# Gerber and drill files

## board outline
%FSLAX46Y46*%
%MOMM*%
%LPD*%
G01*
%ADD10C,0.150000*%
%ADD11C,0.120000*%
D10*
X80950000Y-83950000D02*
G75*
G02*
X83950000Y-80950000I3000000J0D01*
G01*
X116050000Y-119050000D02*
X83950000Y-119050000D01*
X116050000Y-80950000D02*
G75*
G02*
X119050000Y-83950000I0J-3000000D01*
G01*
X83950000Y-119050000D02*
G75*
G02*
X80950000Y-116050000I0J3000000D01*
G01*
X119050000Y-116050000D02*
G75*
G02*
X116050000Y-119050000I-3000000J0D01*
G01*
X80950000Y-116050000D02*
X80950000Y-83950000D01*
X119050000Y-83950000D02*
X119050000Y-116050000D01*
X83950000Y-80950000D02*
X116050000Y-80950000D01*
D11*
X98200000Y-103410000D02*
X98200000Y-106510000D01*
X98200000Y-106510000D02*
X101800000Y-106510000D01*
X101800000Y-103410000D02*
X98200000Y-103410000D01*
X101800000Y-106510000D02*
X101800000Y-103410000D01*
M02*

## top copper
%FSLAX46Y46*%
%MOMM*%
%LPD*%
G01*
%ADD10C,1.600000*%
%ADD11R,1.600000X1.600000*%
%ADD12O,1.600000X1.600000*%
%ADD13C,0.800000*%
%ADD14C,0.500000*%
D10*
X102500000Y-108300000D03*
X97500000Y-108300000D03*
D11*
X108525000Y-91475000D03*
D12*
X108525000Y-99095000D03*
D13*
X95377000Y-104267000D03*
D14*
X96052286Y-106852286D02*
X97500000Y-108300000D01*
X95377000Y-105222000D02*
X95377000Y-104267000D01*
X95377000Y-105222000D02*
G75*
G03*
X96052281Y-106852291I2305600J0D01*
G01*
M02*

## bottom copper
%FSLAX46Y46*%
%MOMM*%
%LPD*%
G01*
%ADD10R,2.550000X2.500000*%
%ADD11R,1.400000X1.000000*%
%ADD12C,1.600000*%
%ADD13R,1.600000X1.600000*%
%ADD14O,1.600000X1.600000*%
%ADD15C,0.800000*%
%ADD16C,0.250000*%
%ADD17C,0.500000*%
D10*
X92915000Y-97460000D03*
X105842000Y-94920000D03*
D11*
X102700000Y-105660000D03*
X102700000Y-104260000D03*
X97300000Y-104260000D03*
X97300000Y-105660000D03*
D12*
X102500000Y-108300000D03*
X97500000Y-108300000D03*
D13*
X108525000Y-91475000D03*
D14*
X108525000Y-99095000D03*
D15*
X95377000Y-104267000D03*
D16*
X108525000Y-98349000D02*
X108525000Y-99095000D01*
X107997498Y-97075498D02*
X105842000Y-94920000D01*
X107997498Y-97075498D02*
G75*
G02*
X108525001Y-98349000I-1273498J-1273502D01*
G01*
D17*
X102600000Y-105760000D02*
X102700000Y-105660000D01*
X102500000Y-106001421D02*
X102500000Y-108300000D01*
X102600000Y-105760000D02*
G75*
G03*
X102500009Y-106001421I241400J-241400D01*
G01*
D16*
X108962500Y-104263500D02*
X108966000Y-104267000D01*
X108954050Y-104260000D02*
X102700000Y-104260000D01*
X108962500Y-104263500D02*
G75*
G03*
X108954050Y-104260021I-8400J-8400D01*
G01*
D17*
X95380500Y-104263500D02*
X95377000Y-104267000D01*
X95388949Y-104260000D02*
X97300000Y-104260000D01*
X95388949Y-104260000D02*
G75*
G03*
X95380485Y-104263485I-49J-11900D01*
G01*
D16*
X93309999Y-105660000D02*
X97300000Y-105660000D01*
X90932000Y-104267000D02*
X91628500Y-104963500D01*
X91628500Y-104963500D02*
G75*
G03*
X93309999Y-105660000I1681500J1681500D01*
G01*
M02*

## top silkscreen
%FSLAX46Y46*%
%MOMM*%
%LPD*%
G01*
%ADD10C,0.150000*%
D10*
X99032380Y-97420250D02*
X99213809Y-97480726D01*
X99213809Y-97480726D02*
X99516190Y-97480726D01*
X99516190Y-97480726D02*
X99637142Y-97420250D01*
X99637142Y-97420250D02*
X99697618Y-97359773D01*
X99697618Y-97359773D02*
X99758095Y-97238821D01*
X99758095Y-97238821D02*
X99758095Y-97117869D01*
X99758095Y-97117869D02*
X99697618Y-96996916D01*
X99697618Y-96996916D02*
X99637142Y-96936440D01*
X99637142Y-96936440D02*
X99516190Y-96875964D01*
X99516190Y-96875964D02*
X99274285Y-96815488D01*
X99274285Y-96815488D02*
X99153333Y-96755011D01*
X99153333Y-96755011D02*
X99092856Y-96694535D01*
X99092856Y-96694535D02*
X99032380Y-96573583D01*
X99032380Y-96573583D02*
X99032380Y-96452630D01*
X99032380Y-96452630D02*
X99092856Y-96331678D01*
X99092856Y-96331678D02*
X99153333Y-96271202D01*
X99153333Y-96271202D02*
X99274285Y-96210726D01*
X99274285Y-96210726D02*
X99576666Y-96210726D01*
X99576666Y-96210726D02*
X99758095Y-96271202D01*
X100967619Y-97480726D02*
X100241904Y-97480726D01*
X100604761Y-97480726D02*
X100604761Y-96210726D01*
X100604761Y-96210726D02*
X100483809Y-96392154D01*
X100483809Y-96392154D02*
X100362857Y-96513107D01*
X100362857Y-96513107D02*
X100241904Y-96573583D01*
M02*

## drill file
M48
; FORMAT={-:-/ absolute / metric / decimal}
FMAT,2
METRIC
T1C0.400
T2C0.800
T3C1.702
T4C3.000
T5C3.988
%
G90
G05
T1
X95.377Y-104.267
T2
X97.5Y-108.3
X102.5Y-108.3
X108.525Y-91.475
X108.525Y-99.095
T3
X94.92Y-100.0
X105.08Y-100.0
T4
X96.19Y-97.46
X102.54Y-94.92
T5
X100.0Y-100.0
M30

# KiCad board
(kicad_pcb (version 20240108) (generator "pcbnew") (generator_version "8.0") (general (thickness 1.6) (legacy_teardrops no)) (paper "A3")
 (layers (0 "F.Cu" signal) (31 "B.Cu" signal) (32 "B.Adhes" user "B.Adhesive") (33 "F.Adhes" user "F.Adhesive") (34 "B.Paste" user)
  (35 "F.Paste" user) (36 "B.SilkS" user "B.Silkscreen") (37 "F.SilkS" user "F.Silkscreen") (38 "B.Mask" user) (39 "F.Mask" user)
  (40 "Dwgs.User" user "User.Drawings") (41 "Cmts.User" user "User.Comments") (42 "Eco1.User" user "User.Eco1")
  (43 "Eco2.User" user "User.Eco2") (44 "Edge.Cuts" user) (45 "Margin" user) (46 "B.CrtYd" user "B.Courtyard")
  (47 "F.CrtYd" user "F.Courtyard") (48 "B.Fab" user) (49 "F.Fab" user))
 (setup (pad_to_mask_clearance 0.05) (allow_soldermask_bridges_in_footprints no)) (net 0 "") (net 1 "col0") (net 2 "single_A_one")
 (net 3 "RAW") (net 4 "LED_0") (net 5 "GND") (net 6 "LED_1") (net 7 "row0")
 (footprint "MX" (layer "F.Cu") (at 100 100)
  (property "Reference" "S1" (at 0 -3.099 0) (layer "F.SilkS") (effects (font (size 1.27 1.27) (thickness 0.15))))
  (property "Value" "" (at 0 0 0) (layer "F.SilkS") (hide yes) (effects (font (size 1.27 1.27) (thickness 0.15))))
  (pad "" np_thru_hole circle (at -5.08 0) (size 1.7018 1.7018) (drill 1.7018) (layers "*.Cu" "*.Mask"))
  (pad "" np_thru_hole circle (at -3.81 -2.54) (size 3 3) (drill 3) (layers "*.Cu" "*.Mask"))
  (pad "" np_thru_hole circle (at 0 0) (size 3.9878 3.9878) (drill 3.9878) (layers "*.Cu" "*.Mask"))
  (pad "" np_thru_hole circle (at 2.54 -5.08) (size 3 3) (drill 3) (layers "*.Cu" "*.Mask"))
  (pad "" np_thru_hole circle (at 5.08 0) (size 1.7018 1.7018) (drill 1.7018) (layers "*.Cu" "*.Mask"))
  (pad "1" smd rect (at -7.085 -2.54) (size 2.55 2.5) (layers "B.Cu" "B.Paste" "B.Mask") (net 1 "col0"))
  (pad "2" smd rect (at 5.842 -5.08) (size 2.55 2.5) (layers "B.Cu" "B.Paste" "B.Mask") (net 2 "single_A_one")))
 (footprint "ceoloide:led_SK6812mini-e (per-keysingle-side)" (layer "B.Cu") (at 100 104.96)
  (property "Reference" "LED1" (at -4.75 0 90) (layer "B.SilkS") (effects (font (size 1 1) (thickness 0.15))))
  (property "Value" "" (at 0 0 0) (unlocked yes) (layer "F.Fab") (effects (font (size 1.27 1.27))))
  (fp_line (start -1.8 -1.55) (end -1.8 1.55) (stroke (width 0.12) (type solid)) (layer "Edge.Cuts"))
  (fp_line (start -1.8 1.55) (end 1.8 1.55) (stroke (width 0.12) (type solid)) (layer "Edge.Cuts"))
  (fp_line (start 1.8 -1.55) (end -1.8 -1.55) (stroke (width 0.12) (type solid)) (layer "Edge.Cuts"))
  (fp_line (start 1.8 1.55) (end 1.8 -1.55) (stroke (width 0.12) (type solid)) (layer "Edge.Cuts"))
  (pad "1" smd rect (at 2.7 0.7) (size 1.4 1) (layers "B.Cu" "B.Paste" "B.Mask") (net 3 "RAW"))
  (pad "2" smd rect (at 2.7 -0.7) (size 1.4 1) (layers "B.Cu" "B.Paste" "B.Mask") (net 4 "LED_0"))
  (pad "3" smd rect (at -2.7 -0.7) (size 1.4 1) (layers "B.Cu" "B.Paste" "B.Mask") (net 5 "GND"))
  (pad "4" smd rect (at -2.7 0.7) (size 1.4 1) (layers "B.Cu" "B.Paste" "B.Mask") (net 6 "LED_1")))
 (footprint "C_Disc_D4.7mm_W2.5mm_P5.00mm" (layer "B.Cu") (at 102.5 108.3 180)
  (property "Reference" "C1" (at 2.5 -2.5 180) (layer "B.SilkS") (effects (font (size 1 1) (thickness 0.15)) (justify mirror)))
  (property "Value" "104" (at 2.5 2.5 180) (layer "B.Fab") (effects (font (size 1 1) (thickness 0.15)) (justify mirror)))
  (pad "1" thru_hole circle (at 0 0) (size 1.6 1.6) (drill 0.8) (layers "*.Cu" "*.Mask") (remove_unused_layers no) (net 3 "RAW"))
  (pad "2" thru_hole circle (at 5 0) (size 1.6 1.6) (drill 0.8) (layers "*.Cu" "*.Mask") (remove_unused_layers no) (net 5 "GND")))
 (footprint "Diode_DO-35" (layer "B.Cu") (at 108.525 91.475 -90)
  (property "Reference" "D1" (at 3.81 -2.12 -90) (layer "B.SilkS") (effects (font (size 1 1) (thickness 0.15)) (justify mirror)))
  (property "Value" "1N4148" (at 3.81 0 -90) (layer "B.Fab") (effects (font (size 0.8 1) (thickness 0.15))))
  (pad "1" thru_hole rect (at 0 0 270) (size 1.6 1.6) (drill 0.8) (layers "*.Cu" "*.Mask") (remove_unused_layers no) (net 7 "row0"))
  (pad "2" thru_hole oval (at 7.62 0 270) (size 1.6 1.6) (drill 0.8) (layers "*.Cu" "*.Mask") (remove_unused_layers no)
   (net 2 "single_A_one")))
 (gr_arc (start 80.95 83.95) (mid 81.82868 81.82868) (end 83.95 80.95) (stroke (width 0.15) (type solid)) (layer "Edge.Cuts"))
 (gr_line (start 116.05 119.05) (end 83.95 119.05) (stroke (width 0.15) (type solid)) (layer "Edge.Cuts"))
 (gr_arc (start 116.05 80.95) (mid 118.17132 81.82868) (end 119.05 83.95) (stroke (width 0.15) (type solid)) (layer "Edge.Cuts"))
 (gr_arc (start 83.95 119.05) (mid 81.82868 118.17132) (end 80.95 116.05) (stroke (width 0.15) (type solid)) (layer "Edge.Cuts"))
 (gr_arc (start 119.05 116.05) (mid 118.17132 118.17132) (end 116.05 119.05) (stroke (width 0.15) (type solid)) (layer "Edge.Cuts"))
 (gr_line (start 80.95 116.05) (end 80.95 83.95) (stroke (width 0.15) (type solid)) (layer "Edge.Cuts"))
 (gr_line (start 119.05 83.95) (end 119.05 116.05) (stroke (width 0.15) (type solid)) (layer "Edge.Cuts"))
 (gr_line (start 83.95 80.95) (end 116.05 80.95) (stroke (width 0.15) (type solid)) (layer "Edge.Cuts"))
 (segment (start 108.525 98.349) (end 108.525 99.095) (width 0.25) (layer "B.Cu") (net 2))
 (segment (start 107.997498 97.075498) (end 105.842 94.92) (width 0.25) (layer "B.Cu") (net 2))
 (arc (start 107.997498 97.075498) (mid 108.387906 97.659785) (end 108.525 98.349) (width 0.25) (layer "B.Cu") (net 2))
 (segment (start 102.6 105.76) (end 102.7 105.66) (width 0.5) (layer "B.Cu") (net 3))
 (segment (start 102.5 106.001421) (end 102.5 108.3) (width 0.5) (layer "B.Cu") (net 3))
 (arc (start 102.6 105.76) (mid 102.525989 105.870764) (end 102.5 106.001421) (width 0.5) (layer "B.Cu") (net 3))
 (segment (start 108.9625 104.2635) (end 108.966 104.267) (width 0.25) (layer "B.Cu") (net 4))
 (segment (start 108.95405 104.26) (end 102.7 104.26) (width 0.25) (layer "B.Cu") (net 4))
 (arc (start 108.9625 104.2635) (mid 108.958623 104.260909) (end 108.95405 104.26) (width 0.25) (layer "B.Cu") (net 4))
 (segment (start 96.052286 106.852286) (end 97.5 108.3) (width 0.5) (layer "F.Cu") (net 5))
 (segment (start 95.377 105.222) (end 95.377 104.267) (width 0.5) (layer "F.Cu") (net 5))
 (via (at 95.377 104.267) (size 0.8) (drill 0.4) (layers "F.Cu" "B.Cu") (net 5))
 (arc (start 95.377 105.222) (mid 95.552501 106.104304) (end 96.052286 106.852286) (width 0.5) (layer "F.Cu") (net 5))
 (segment (start 95.3805 104.2635) (end 95.377 104.267) (width 0.5) (layer "B.Cu") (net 5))
 (segment (start 95.388949 104.26) (end 97.3 104.26) (width 0.5) (layer "B.Cu") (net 5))
 (arc (start 95.388949 104.26) (mid 95.384376 104.260909) (end 95.3805 104.2635) (width 0.5) (layer "B.Cu") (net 5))
 (segment (start 93.309999 105.66) (end 97.3 105.66) (width 0.25) (layer "B.Cu") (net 6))
 (segment (start 90.932 104.267) (end 91.6285 104.9635) (width 0.25) (layer "B.Cu") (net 6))
 (arc (start 91.6285 104.9635) (mid 92.399978 105.478985) (end 93.309999 105.66) (width 0.25) (layer "B.Cu") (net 6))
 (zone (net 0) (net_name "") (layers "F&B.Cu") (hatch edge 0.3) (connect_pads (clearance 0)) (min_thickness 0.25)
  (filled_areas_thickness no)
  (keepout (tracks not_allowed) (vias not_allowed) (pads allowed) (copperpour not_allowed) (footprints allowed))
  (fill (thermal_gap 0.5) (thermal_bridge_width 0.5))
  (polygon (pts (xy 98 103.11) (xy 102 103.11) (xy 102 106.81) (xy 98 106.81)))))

